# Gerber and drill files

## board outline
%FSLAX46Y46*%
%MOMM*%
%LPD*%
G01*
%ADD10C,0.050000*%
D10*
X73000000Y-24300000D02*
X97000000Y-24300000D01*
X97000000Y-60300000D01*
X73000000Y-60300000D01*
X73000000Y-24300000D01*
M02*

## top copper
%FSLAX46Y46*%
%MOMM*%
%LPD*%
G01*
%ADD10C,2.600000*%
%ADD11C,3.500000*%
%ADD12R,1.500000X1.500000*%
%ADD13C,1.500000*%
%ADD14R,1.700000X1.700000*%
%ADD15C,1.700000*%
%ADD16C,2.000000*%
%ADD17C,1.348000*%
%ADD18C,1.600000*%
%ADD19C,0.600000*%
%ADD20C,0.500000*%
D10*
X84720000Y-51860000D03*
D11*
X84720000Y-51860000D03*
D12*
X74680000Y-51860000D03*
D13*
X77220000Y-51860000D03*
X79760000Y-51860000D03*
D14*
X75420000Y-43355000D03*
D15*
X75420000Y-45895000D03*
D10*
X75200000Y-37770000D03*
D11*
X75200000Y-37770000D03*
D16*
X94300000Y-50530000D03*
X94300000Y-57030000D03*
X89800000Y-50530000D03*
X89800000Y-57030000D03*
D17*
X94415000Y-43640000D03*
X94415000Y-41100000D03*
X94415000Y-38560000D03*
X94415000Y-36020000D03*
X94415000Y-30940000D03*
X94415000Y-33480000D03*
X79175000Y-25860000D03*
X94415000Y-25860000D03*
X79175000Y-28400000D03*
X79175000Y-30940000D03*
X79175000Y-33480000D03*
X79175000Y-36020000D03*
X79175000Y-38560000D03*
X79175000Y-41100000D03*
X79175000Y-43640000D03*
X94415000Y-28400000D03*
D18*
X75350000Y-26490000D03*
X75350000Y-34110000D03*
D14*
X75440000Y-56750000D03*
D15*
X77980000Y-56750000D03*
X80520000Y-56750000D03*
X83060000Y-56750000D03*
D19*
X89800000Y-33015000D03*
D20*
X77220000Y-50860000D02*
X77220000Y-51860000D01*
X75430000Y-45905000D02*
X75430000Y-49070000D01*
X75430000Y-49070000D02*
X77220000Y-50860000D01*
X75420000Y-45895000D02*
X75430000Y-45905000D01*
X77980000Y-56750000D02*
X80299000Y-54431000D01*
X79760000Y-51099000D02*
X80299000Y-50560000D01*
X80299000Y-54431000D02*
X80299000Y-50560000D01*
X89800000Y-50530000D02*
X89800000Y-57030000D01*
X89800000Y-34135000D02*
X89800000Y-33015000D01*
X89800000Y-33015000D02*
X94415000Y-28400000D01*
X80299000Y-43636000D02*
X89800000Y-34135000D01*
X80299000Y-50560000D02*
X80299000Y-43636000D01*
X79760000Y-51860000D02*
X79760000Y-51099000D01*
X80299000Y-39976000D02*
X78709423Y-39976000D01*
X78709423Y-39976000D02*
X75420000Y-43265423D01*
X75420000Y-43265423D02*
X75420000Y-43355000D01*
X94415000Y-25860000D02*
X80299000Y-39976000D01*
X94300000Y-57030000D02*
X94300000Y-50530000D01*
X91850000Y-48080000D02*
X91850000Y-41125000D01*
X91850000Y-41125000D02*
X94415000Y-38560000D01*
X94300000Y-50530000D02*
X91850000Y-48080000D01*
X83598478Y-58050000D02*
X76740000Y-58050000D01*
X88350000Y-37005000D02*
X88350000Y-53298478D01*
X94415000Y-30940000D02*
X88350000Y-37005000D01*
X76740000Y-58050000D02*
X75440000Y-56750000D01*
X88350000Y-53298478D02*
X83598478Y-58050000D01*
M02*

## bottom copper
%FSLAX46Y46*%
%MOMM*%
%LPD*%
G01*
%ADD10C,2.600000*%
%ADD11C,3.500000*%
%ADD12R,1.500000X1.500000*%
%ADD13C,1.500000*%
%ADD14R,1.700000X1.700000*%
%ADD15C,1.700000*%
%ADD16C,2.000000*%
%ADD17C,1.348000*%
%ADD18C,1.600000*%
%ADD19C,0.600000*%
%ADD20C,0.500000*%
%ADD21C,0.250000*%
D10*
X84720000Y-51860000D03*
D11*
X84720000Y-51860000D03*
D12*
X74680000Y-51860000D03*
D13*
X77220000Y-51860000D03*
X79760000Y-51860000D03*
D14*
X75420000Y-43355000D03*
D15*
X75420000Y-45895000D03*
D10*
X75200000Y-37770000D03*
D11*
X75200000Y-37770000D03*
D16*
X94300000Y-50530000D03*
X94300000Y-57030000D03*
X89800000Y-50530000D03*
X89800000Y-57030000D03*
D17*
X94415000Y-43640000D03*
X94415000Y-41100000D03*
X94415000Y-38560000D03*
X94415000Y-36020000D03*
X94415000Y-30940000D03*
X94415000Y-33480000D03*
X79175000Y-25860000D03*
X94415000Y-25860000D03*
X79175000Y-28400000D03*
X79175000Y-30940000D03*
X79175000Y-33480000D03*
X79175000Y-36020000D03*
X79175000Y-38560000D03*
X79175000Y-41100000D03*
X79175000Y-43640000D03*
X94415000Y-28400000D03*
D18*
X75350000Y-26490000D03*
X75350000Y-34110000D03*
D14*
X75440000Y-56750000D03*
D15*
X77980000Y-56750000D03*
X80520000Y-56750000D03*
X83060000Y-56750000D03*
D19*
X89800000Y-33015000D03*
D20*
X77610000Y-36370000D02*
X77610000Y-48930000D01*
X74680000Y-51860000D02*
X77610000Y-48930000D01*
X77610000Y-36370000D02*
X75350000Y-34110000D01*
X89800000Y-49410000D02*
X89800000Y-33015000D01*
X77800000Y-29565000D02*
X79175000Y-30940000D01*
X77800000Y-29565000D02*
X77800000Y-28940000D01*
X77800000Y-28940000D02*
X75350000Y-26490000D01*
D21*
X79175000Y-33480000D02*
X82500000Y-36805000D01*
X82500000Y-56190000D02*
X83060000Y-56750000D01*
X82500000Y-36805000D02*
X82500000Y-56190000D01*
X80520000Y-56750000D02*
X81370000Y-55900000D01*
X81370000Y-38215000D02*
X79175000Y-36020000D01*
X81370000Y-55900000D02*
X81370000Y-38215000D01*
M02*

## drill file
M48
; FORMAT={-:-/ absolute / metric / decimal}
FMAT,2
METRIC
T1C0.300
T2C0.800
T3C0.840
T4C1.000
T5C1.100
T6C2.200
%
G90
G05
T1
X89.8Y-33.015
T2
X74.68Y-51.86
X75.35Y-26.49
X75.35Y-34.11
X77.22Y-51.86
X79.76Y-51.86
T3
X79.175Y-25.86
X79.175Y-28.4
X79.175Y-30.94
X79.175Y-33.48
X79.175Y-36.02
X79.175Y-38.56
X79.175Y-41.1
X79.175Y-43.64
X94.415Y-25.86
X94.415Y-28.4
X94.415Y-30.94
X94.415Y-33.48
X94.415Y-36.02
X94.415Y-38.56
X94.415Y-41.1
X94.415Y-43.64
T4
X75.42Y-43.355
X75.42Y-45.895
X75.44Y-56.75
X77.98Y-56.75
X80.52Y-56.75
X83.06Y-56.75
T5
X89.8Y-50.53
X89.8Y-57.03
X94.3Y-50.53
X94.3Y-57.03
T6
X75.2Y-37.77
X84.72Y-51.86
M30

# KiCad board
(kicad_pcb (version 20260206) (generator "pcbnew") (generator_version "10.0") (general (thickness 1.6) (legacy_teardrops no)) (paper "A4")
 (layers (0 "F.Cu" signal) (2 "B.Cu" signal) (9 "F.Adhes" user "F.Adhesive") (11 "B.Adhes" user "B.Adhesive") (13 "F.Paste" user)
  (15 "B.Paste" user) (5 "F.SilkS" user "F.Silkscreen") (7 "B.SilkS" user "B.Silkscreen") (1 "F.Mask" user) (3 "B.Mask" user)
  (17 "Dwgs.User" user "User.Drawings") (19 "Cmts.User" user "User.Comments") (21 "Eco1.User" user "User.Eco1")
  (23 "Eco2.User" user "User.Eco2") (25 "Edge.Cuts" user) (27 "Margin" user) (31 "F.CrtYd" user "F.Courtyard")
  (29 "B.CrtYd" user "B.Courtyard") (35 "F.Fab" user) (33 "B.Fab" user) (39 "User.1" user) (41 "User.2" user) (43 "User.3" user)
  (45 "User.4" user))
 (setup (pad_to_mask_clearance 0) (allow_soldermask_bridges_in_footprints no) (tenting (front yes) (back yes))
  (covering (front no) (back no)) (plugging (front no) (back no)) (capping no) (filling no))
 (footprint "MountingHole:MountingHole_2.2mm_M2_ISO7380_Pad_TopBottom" (layer "F.Cu") (at 84.72 51.86)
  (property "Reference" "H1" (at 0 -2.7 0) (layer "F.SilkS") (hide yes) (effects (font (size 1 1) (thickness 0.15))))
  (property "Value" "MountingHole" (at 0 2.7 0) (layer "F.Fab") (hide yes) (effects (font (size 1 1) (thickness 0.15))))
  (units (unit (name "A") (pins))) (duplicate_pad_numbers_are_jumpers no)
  (pad "1" thru_hole circle (at 0 0) (size 2.6 2.6) (drill 2.2) (layers "*.Cu" "*.Mask") (remove_unused_layers no) (zone_connect 2))
  (pad "1" connect circle (at 0 0) (size 3.5 3.5) (layers "F.Cu" "F.Mask") (zone_connect 2))
  (pad "1" connect circle (at 0 0) (size 3.5 3.5) (layers "B.Cu" "B.Mask") (zone_connect 2)))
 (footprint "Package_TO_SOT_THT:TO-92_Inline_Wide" (layer "F.Cu") (at 74.68 51.86)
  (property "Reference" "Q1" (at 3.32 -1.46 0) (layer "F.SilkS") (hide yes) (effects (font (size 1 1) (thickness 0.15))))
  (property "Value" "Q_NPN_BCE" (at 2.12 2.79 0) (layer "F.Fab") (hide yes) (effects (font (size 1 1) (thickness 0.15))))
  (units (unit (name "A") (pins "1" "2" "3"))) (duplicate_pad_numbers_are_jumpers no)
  (pad "1" thru_hole rect (at 0 0) (size 1.5 1.5) (drill 0.8) (layers "*.Cu" "*.Mask") (remove_unused_layers no) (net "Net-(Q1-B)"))
  (pad "2" thru_hole circle (at 2.54 0) (size 1.5 1.5) (drill 0.8) (layers "*.Cu" "*.Mask") (remove_unused_layers no) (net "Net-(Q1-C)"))
  (pad "3" thru_hole circle (at 5.08 0) (size 1.5 1.5) (drill 0.8) (layers "*.Cu" "*.Mask") (remove_unused_layers no) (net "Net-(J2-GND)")))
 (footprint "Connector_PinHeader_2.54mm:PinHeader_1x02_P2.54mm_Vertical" (layer "F.Cu") (at 75.42 43.355)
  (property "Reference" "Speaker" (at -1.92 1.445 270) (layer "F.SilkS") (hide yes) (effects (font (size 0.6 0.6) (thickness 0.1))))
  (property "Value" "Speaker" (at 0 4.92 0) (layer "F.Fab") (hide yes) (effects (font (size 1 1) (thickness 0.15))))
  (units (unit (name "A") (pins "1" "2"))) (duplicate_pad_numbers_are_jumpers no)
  (pad "1" thru_hole rect (at 0 0) (size 1.7 1.7) (drill 1) (layers "*.Cu" "*.Mask") (remove_unused_layers no) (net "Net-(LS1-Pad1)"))
  (pad "2" thru_hole circle (at 0 2.54) (size 1.7 1.7) (drill 1) (layers "*.Cu" "*.Mask") (remove_unused_layers no) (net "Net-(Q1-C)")))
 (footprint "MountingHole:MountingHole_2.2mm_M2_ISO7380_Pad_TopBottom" (layer "F.Cu") (at 75.2 37.77)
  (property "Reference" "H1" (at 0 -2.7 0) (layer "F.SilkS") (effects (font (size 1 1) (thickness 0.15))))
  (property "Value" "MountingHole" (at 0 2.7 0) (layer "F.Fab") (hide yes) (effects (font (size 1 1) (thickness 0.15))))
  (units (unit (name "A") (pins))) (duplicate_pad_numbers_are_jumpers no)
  (pad "1" thru_hole circle (at 0 0) (size 2.6 2.6) (drill 2.2) (layers "*.Cu" "*.Mask") (remove_unused_layers no) (zone_connect 2))
  (pad "1" connect circle (at 0 0) (size 3.5 3.5) (layers "F.Cu" "F.Mask") (zone_connect 2))
  (pad "1" connect circle (at 0 0) (size 3.5 3.5) (layers "B.Cu" "B.Mask") (zone_connect 2)))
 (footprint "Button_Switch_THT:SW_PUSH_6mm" (layer "F.Cu") (at 94.3 50.53 -90)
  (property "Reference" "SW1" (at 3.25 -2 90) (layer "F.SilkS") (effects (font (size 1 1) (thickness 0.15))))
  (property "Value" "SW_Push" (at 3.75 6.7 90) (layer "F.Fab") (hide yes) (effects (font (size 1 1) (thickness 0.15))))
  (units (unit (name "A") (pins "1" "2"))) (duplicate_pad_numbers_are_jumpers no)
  (pad "1" thru_hole circle (at 0 0) (size 2 2) (drill 1.1) (layers "*.Cu" "*.Mask") (remove_unused_layers no) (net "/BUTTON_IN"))
  (pad "1" thru_hole circle (at 6.5 0) (size 2 2) (drill 1.1) (layers "*.Cu" "*.Mask") (remove_unused_layers no) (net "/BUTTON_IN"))
  (pad "2" thru_hole circle (at 0 4.5) (size 2 2) (drill 1.1) (layers "*.Cu" "*.Mask") (remove_unused_layers no) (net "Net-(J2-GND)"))
  (pad "2" thru_hole circle (at 6.5 4.5) (size 2 2) (drill 1.1) (layers "*.Cu" "*.Mask") (remove_unused_layers no) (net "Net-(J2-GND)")))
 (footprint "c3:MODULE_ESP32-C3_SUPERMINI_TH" (layer "F.Cu") (at 86.795 35.76)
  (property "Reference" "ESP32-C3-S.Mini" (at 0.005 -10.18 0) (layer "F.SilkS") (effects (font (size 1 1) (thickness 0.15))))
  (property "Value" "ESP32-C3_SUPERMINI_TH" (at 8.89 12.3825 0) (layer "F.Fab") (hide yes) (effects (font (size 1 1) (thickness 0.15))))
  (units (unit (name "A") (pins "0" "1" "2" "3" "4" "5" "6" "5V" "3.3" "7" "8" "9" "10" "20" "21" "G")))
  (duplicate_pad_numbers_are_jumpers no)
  (pad "0" thru_hole circle (at 7.62 7.88) (size 1.348 1.348) (drill 0.84) (layers "*.Cu" "*.Mask") (remove_unused_layers no)
   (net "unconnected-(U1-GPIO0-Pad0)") (solder_mask_margin 0.102))
  (pad "1" thru_hole circle (at 7.62 5.34) (size 1.348 1.348) (drill 0.84) (layers "*.Cu" "*.Mask") (remove_unused_layers no)
   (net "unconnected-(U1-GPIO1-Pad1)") (solder_mask_margin 0.102))
  (pad "2" thru_hole circle (at 7.62 2.8) (size 1.348 1.348) (drill 0.84) (layers "*.Cu" "*.Mask") (remove_unused_layers no)
   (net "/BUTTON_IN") (solder_mask_margin 0.102))
  (pad "3" thru_hole circle (at 7.62 0.26) (size 1.348 1.348) (drill 0.84) (layers "*.Cu" "*.Mask") (remove_unused_layers no)
   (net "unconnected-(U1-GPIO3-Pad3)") (solder_mask_margin 0.102))
  (pad "3.3" thru_hole circle (at 7.62 -4.82) (size 1.348 1.348) (drill 0.84) (layers "*.Cu" "*.Mask") (remove_unused_layers no)
   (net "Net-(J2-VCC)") (solder_mask_margin 0.102))
  (pad "4" thru_hole circle (at 7.62 -2.28) (size 1.348 1.348) (drill 0.84) (layers "*.Cu" "*.Mask") (remove_unused_layers no)
   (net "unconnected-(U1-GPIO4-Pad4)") (solder_mask_margin 0.102))
  (pad "5" thru_hole circle (at -7.62 -9.9) (size 1.348 1.348) (drill 0.84) (layers "*.Cu" "*.Mask") (remove_unused_layers no)
   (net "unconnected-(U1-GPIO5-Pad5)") (solder_mask_margin 0.102))
  (pad "5V" thru_hole circle (at 7.62 -9.9) (size 1.348 1.348) (drill 0.84) (layers "*.Cu" "*.Mask") (remove_unused_layers no)
   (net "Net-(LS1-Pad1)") (solder_mask_margin 0.102))
  (pad "6" thru_hole circle (at -7.62 -7.36) (size 1.348 1.348) (drill 0.84) (layers "*.Cu" "*.Mask") (remove_unused_layers no)
   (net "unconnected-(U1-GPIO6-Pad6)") (solder_mask_margin 0.102))
  (pad "7" thru_hole circle (at -7.62 -4.82) (size 1.348 1.348) (drill 0.84) (layers "*.Cu" "*.Mask") (remove_unused_layers no)
   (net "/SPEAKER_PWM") (solder_mask_margin 0.102))
  (pad "8" thru_hole circle (at -7.62 -2.28) (size 1.348 1.348) (drill 0.84) (layers "*.Cu" "*.Mask") (remove_unused_layers no)
   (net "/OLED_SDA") (solder_mask_margin 0.102))
  (pad "9" thru_hole circle (at -7.62 0.26) (size 1.348 1.348) (drill 0.84) (layers "*.Cu" "*.Mask") (remove_unused_layers no)
   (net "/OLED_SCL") (solder_mask_margin 0.102))
  (pad "10" thru_hole circle (at -7.62 2.8) (size 1.348 1.348) (drill 0.84) (layers "*.Cu" "*.Mask") (remove_unused_layers no)
   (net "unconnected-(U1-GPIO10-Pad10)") (solder_mask_margin 0.102))
  (pad "20" thru_hole circle (at -7.62 5.34) (size 1.348 1.348) (drill 0.84) (layers "*.Cu" "*.Mask") (remove_unused_layers no)
   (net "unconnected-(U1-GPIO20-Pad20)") (solder_mask_margin 0.102))
  (pad "21" thru_hole circle (at -7.62 7.88) (size 1.348 1.348) (drill 0.84) (layers "*.Cu" "*.Mask") (remove_unused_layers no)
   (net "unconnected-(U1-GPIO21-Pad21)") (solder_mask_margin 0.102))
  (pad "G" thru_hole circle (at 7.62 -7.36) (size 1.348 1.348) (drill 0.84) (layers "*.Cu" "*.Mask") (remove_unused_layers no)
   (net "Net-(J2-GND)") (solder_mask_margin 0.102)))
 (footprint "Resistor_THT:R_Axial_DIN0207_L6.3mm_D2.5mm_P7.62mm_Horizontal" (layer "F.Cu") (at 75.35 26.49 -90)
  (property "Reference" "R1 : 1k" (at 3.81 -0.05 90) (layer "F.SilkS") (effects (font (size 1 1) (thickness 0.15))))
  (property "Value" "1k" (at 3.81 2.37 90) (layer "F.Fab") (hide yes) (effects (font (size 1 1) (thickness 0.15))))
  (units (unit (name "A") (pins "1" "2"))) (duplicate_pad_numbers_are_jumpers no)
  (pad "1" thru_hole circle (at 0 0 270) (size 1.6 1.6) (drill 0.8) (layers "*.Cu" "*.Mask") (remove_unused_layers no) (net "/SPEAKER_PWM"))
  (pad "2" thru_hole circle (at 7.62 0 270) (size 1.6 1.6) (drill 0.8) (layers "*.Cu" "*.Mask") (remove_unused_layers no) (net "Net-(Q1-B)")))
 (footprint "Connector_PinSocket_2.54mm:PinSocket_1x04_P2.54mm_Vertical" (layer "F.Cu") (at 75.44 56.75 90)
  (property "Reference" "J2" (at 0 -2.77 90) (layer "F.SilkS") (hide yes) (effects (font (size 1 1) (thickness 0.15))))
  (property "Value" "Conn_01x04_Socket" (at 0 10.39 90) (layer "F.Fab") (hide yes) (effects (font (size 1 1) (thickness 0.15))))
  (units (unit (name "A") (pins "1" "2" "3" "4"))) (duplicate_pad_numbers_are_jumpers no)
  (pad "1" thru_hole rect (at 0 0 90) (size 1.7 1.7) (drill 1) (layers "*.Cu" "*.Mask") (remove_unused_layers no) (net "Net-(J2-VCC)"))
  (pad "2" thru_hole circle (at 0 2.54 90) (size 1.7 1.7) (drill 1) (layers "*.Cu" "*.Mask") (remove_unused_layers no) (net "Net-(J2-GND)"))
  (pad "3" thru_hole circle (at 0 5.08 90) (size 1.7 1.7) (drill 1) (layers "*.Cu" "*.Mask") (remove_unused_layers no) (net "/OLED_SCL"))
  (pad "4" thru_hole circle (at 0 7.62 90) (size 1.7 1.7) (drill 1) (layers "*.Cu" "*.Mask") (remove_unused_layers no) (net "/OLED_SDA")))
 (gr_rect (start 73 24.3) (end 97 60.3) (stroke (width 0.05) (type default)) (fill no) (layer "Edge.Cuts"))
 (segment (start 77.61 36.37) (end 77.61 48.93) (width 0.5) (layer "B.Cu") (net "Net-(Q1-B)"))
 (segment (start 74.68 51.86) (end 77.61 48.93) (width 0.5) (layer "B.Cu") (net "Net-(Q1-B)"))
 (segment (start 77.61 36.37) (end 75.35 34.11) (width 0.5) (layer "B.Cu") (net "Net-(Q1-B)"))
 (segment (start 77.22 50.86) (end 77.22 51.86) (width 0.5) (layer "F.Cu") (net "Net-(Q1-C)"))
 (segment (start 75.43 45.905) (end 75.43 49.07) (width 0.5) (layer "F.Cu") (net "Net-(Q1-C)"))
 (segment (start 75.43 49.07) (end 77.22 50.86) (width 0.5) (layer "F.Cu") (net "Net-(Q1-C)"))
 (segment (start 75.42 45.895) (end 75.43 45.905) (width 0.5) (layer "F.Cu") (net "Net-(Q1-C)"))
 (segment (start 77.98 56.75) (end 80.299 54.431) (width 0.5) (layer "F.Cu") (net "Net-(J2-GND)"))
 (segment (start 79.76 51.099) (end 80.299 50.56) (width 0.5) (layer "F.Cu") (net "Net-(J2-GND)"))
 (segment (start 80.299 54.431) (end 80.299 50.56) (width 0.5) (layer "F.Cu") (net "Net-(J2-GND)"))
 (segment (start 89.8 50.53) (end 89.8 57.03) (width 0.5) (layer "F.Cu") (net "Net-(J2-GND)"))
 (segment (start 89.8 34.135) (end 89.8 33.015) (width 0.5) (layer "F.Cu") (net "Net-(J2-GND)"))
 (segment (start 89.8 33.015) (end 94.415 28.4) (width 0.5) (layer "F.Cu") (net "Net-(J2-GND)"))
 (segment (start 80.299 43.636) (end 89.8 34.135) (width 0.5) (layer "F.Cu") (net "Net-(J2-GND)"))
 (segment (start 80.299 50.56) (end 80.299 43.636) (width 0.5) (layer "F.Cu") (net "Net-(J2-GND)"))
 (segment (start 79.76 51.86) (end 79.76 51.099) (width 0.5) (layer "F.Cu") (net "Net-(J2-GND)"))
 (via (at 89.8 33.015) (size 0.6) (drill 0.3) (layers "F.Cu" "B.Cu") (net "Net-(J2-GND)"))
 (segment (start 89.8 49.41) (end 89.8 33.015) (width 0.5) (layer "B.Cu") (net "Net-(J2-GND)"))
 (segment (start 80.299 39.976) (end 78.709423 39.976) (width 0.5) (layer "F.Cu") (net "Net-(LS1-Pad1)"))
 (segment (start 78.709423 39.976) (end 75.42 43.265423) (width 0.5) (layer "F.Cu") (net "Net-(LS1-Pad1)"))
 (segment (start 75.42 43.265423) (end 75.42 43.355) (width 0.5) (layer "F.Cu") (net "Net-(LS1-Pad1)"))
 (segment (start 94.415 25.86) (end 80.299 39.976) (width 0.5) (layer "F.Cu") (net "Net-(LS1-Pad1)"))
 (segment (start 94.3 57.03) (end 94.3 50.53) (width 0.5) (layer "F.Cu") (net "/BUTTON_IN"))
 (segment (start 91.85 48.08) (end 91.85 41.125) (width 0.5) (layer "F.Cu") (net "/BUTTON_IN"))
 (segment (start 91.85 41.125) (end 94.415 38.56) (width 0.5) (layer "F.Cu") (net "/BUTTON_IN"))
 (segment (start 94.3 50.53) (end 91.85 48.08) (width 0.5) (layer "F.Cu") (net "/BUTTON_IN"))
 (segment (start 83.598478 58.05) (end 76.74 58.05) (width 0.5) (layer "F.Cu") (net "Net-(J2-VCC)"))
 (segment (start 88.35 37.005) (end 88.35 53.298478) (width 0.5) (layer "F.Cu") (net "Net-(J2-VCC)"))
 (segment (start 94.415 30.94) (end 88.35 37.005) (width 0.5) (layer "F.Cu") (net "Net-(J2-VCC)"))
 (segment (start 76.74 58.05) (end 75.44 56.75) (width 0.5) (layer "F.Cu") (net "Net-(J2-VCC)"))
 (segment (start 88.35 53.298478) (end 83.598478 58.05) (width 0.5) (layer "F.Cu") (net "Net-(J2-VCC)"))
 (segment (start 77.8 29.565) (end 79.175 30.94) (width 0.5) (layer "B.Cu") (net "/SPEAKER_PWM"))
 (segment (start 77.8 29.565) (end 77.8 28.94) (width 0.5) (layer "B.Cu") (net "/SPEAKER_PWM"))
 (segment (start 77.8 28.94) (end 75.35 26.49) (width 0.5) (layer "B.Cu") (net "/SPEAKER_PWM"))
 (segment (start 79.175 33.48) (end 82.5 36.805) (width 0.25) (layer "B.Cu") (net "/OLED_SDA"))
 (segment (start 82.5 56.19) (end 83.06 56.75) (width 0.25) (layer "B.Cu") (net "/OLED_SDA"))
 (segment (start 82.5 36.805) (end 82.5 56.19) (width 0.25) (layer "B.Cu") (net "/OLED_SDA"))
 (segment (start 80.52 56.75) (end 81.37 55.9) (width 0.25) (layer "B.Cu") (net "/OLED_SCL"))
 (segment (start 81.37 38.215) (end 79.175 36.02) (width 0.25) (layer "B.Cu") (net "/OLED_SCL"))
 (segment (start 81.37 55.9) (end 81.37 38.215) (width 0.25) (layer "B.Cu") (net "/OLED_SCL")))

